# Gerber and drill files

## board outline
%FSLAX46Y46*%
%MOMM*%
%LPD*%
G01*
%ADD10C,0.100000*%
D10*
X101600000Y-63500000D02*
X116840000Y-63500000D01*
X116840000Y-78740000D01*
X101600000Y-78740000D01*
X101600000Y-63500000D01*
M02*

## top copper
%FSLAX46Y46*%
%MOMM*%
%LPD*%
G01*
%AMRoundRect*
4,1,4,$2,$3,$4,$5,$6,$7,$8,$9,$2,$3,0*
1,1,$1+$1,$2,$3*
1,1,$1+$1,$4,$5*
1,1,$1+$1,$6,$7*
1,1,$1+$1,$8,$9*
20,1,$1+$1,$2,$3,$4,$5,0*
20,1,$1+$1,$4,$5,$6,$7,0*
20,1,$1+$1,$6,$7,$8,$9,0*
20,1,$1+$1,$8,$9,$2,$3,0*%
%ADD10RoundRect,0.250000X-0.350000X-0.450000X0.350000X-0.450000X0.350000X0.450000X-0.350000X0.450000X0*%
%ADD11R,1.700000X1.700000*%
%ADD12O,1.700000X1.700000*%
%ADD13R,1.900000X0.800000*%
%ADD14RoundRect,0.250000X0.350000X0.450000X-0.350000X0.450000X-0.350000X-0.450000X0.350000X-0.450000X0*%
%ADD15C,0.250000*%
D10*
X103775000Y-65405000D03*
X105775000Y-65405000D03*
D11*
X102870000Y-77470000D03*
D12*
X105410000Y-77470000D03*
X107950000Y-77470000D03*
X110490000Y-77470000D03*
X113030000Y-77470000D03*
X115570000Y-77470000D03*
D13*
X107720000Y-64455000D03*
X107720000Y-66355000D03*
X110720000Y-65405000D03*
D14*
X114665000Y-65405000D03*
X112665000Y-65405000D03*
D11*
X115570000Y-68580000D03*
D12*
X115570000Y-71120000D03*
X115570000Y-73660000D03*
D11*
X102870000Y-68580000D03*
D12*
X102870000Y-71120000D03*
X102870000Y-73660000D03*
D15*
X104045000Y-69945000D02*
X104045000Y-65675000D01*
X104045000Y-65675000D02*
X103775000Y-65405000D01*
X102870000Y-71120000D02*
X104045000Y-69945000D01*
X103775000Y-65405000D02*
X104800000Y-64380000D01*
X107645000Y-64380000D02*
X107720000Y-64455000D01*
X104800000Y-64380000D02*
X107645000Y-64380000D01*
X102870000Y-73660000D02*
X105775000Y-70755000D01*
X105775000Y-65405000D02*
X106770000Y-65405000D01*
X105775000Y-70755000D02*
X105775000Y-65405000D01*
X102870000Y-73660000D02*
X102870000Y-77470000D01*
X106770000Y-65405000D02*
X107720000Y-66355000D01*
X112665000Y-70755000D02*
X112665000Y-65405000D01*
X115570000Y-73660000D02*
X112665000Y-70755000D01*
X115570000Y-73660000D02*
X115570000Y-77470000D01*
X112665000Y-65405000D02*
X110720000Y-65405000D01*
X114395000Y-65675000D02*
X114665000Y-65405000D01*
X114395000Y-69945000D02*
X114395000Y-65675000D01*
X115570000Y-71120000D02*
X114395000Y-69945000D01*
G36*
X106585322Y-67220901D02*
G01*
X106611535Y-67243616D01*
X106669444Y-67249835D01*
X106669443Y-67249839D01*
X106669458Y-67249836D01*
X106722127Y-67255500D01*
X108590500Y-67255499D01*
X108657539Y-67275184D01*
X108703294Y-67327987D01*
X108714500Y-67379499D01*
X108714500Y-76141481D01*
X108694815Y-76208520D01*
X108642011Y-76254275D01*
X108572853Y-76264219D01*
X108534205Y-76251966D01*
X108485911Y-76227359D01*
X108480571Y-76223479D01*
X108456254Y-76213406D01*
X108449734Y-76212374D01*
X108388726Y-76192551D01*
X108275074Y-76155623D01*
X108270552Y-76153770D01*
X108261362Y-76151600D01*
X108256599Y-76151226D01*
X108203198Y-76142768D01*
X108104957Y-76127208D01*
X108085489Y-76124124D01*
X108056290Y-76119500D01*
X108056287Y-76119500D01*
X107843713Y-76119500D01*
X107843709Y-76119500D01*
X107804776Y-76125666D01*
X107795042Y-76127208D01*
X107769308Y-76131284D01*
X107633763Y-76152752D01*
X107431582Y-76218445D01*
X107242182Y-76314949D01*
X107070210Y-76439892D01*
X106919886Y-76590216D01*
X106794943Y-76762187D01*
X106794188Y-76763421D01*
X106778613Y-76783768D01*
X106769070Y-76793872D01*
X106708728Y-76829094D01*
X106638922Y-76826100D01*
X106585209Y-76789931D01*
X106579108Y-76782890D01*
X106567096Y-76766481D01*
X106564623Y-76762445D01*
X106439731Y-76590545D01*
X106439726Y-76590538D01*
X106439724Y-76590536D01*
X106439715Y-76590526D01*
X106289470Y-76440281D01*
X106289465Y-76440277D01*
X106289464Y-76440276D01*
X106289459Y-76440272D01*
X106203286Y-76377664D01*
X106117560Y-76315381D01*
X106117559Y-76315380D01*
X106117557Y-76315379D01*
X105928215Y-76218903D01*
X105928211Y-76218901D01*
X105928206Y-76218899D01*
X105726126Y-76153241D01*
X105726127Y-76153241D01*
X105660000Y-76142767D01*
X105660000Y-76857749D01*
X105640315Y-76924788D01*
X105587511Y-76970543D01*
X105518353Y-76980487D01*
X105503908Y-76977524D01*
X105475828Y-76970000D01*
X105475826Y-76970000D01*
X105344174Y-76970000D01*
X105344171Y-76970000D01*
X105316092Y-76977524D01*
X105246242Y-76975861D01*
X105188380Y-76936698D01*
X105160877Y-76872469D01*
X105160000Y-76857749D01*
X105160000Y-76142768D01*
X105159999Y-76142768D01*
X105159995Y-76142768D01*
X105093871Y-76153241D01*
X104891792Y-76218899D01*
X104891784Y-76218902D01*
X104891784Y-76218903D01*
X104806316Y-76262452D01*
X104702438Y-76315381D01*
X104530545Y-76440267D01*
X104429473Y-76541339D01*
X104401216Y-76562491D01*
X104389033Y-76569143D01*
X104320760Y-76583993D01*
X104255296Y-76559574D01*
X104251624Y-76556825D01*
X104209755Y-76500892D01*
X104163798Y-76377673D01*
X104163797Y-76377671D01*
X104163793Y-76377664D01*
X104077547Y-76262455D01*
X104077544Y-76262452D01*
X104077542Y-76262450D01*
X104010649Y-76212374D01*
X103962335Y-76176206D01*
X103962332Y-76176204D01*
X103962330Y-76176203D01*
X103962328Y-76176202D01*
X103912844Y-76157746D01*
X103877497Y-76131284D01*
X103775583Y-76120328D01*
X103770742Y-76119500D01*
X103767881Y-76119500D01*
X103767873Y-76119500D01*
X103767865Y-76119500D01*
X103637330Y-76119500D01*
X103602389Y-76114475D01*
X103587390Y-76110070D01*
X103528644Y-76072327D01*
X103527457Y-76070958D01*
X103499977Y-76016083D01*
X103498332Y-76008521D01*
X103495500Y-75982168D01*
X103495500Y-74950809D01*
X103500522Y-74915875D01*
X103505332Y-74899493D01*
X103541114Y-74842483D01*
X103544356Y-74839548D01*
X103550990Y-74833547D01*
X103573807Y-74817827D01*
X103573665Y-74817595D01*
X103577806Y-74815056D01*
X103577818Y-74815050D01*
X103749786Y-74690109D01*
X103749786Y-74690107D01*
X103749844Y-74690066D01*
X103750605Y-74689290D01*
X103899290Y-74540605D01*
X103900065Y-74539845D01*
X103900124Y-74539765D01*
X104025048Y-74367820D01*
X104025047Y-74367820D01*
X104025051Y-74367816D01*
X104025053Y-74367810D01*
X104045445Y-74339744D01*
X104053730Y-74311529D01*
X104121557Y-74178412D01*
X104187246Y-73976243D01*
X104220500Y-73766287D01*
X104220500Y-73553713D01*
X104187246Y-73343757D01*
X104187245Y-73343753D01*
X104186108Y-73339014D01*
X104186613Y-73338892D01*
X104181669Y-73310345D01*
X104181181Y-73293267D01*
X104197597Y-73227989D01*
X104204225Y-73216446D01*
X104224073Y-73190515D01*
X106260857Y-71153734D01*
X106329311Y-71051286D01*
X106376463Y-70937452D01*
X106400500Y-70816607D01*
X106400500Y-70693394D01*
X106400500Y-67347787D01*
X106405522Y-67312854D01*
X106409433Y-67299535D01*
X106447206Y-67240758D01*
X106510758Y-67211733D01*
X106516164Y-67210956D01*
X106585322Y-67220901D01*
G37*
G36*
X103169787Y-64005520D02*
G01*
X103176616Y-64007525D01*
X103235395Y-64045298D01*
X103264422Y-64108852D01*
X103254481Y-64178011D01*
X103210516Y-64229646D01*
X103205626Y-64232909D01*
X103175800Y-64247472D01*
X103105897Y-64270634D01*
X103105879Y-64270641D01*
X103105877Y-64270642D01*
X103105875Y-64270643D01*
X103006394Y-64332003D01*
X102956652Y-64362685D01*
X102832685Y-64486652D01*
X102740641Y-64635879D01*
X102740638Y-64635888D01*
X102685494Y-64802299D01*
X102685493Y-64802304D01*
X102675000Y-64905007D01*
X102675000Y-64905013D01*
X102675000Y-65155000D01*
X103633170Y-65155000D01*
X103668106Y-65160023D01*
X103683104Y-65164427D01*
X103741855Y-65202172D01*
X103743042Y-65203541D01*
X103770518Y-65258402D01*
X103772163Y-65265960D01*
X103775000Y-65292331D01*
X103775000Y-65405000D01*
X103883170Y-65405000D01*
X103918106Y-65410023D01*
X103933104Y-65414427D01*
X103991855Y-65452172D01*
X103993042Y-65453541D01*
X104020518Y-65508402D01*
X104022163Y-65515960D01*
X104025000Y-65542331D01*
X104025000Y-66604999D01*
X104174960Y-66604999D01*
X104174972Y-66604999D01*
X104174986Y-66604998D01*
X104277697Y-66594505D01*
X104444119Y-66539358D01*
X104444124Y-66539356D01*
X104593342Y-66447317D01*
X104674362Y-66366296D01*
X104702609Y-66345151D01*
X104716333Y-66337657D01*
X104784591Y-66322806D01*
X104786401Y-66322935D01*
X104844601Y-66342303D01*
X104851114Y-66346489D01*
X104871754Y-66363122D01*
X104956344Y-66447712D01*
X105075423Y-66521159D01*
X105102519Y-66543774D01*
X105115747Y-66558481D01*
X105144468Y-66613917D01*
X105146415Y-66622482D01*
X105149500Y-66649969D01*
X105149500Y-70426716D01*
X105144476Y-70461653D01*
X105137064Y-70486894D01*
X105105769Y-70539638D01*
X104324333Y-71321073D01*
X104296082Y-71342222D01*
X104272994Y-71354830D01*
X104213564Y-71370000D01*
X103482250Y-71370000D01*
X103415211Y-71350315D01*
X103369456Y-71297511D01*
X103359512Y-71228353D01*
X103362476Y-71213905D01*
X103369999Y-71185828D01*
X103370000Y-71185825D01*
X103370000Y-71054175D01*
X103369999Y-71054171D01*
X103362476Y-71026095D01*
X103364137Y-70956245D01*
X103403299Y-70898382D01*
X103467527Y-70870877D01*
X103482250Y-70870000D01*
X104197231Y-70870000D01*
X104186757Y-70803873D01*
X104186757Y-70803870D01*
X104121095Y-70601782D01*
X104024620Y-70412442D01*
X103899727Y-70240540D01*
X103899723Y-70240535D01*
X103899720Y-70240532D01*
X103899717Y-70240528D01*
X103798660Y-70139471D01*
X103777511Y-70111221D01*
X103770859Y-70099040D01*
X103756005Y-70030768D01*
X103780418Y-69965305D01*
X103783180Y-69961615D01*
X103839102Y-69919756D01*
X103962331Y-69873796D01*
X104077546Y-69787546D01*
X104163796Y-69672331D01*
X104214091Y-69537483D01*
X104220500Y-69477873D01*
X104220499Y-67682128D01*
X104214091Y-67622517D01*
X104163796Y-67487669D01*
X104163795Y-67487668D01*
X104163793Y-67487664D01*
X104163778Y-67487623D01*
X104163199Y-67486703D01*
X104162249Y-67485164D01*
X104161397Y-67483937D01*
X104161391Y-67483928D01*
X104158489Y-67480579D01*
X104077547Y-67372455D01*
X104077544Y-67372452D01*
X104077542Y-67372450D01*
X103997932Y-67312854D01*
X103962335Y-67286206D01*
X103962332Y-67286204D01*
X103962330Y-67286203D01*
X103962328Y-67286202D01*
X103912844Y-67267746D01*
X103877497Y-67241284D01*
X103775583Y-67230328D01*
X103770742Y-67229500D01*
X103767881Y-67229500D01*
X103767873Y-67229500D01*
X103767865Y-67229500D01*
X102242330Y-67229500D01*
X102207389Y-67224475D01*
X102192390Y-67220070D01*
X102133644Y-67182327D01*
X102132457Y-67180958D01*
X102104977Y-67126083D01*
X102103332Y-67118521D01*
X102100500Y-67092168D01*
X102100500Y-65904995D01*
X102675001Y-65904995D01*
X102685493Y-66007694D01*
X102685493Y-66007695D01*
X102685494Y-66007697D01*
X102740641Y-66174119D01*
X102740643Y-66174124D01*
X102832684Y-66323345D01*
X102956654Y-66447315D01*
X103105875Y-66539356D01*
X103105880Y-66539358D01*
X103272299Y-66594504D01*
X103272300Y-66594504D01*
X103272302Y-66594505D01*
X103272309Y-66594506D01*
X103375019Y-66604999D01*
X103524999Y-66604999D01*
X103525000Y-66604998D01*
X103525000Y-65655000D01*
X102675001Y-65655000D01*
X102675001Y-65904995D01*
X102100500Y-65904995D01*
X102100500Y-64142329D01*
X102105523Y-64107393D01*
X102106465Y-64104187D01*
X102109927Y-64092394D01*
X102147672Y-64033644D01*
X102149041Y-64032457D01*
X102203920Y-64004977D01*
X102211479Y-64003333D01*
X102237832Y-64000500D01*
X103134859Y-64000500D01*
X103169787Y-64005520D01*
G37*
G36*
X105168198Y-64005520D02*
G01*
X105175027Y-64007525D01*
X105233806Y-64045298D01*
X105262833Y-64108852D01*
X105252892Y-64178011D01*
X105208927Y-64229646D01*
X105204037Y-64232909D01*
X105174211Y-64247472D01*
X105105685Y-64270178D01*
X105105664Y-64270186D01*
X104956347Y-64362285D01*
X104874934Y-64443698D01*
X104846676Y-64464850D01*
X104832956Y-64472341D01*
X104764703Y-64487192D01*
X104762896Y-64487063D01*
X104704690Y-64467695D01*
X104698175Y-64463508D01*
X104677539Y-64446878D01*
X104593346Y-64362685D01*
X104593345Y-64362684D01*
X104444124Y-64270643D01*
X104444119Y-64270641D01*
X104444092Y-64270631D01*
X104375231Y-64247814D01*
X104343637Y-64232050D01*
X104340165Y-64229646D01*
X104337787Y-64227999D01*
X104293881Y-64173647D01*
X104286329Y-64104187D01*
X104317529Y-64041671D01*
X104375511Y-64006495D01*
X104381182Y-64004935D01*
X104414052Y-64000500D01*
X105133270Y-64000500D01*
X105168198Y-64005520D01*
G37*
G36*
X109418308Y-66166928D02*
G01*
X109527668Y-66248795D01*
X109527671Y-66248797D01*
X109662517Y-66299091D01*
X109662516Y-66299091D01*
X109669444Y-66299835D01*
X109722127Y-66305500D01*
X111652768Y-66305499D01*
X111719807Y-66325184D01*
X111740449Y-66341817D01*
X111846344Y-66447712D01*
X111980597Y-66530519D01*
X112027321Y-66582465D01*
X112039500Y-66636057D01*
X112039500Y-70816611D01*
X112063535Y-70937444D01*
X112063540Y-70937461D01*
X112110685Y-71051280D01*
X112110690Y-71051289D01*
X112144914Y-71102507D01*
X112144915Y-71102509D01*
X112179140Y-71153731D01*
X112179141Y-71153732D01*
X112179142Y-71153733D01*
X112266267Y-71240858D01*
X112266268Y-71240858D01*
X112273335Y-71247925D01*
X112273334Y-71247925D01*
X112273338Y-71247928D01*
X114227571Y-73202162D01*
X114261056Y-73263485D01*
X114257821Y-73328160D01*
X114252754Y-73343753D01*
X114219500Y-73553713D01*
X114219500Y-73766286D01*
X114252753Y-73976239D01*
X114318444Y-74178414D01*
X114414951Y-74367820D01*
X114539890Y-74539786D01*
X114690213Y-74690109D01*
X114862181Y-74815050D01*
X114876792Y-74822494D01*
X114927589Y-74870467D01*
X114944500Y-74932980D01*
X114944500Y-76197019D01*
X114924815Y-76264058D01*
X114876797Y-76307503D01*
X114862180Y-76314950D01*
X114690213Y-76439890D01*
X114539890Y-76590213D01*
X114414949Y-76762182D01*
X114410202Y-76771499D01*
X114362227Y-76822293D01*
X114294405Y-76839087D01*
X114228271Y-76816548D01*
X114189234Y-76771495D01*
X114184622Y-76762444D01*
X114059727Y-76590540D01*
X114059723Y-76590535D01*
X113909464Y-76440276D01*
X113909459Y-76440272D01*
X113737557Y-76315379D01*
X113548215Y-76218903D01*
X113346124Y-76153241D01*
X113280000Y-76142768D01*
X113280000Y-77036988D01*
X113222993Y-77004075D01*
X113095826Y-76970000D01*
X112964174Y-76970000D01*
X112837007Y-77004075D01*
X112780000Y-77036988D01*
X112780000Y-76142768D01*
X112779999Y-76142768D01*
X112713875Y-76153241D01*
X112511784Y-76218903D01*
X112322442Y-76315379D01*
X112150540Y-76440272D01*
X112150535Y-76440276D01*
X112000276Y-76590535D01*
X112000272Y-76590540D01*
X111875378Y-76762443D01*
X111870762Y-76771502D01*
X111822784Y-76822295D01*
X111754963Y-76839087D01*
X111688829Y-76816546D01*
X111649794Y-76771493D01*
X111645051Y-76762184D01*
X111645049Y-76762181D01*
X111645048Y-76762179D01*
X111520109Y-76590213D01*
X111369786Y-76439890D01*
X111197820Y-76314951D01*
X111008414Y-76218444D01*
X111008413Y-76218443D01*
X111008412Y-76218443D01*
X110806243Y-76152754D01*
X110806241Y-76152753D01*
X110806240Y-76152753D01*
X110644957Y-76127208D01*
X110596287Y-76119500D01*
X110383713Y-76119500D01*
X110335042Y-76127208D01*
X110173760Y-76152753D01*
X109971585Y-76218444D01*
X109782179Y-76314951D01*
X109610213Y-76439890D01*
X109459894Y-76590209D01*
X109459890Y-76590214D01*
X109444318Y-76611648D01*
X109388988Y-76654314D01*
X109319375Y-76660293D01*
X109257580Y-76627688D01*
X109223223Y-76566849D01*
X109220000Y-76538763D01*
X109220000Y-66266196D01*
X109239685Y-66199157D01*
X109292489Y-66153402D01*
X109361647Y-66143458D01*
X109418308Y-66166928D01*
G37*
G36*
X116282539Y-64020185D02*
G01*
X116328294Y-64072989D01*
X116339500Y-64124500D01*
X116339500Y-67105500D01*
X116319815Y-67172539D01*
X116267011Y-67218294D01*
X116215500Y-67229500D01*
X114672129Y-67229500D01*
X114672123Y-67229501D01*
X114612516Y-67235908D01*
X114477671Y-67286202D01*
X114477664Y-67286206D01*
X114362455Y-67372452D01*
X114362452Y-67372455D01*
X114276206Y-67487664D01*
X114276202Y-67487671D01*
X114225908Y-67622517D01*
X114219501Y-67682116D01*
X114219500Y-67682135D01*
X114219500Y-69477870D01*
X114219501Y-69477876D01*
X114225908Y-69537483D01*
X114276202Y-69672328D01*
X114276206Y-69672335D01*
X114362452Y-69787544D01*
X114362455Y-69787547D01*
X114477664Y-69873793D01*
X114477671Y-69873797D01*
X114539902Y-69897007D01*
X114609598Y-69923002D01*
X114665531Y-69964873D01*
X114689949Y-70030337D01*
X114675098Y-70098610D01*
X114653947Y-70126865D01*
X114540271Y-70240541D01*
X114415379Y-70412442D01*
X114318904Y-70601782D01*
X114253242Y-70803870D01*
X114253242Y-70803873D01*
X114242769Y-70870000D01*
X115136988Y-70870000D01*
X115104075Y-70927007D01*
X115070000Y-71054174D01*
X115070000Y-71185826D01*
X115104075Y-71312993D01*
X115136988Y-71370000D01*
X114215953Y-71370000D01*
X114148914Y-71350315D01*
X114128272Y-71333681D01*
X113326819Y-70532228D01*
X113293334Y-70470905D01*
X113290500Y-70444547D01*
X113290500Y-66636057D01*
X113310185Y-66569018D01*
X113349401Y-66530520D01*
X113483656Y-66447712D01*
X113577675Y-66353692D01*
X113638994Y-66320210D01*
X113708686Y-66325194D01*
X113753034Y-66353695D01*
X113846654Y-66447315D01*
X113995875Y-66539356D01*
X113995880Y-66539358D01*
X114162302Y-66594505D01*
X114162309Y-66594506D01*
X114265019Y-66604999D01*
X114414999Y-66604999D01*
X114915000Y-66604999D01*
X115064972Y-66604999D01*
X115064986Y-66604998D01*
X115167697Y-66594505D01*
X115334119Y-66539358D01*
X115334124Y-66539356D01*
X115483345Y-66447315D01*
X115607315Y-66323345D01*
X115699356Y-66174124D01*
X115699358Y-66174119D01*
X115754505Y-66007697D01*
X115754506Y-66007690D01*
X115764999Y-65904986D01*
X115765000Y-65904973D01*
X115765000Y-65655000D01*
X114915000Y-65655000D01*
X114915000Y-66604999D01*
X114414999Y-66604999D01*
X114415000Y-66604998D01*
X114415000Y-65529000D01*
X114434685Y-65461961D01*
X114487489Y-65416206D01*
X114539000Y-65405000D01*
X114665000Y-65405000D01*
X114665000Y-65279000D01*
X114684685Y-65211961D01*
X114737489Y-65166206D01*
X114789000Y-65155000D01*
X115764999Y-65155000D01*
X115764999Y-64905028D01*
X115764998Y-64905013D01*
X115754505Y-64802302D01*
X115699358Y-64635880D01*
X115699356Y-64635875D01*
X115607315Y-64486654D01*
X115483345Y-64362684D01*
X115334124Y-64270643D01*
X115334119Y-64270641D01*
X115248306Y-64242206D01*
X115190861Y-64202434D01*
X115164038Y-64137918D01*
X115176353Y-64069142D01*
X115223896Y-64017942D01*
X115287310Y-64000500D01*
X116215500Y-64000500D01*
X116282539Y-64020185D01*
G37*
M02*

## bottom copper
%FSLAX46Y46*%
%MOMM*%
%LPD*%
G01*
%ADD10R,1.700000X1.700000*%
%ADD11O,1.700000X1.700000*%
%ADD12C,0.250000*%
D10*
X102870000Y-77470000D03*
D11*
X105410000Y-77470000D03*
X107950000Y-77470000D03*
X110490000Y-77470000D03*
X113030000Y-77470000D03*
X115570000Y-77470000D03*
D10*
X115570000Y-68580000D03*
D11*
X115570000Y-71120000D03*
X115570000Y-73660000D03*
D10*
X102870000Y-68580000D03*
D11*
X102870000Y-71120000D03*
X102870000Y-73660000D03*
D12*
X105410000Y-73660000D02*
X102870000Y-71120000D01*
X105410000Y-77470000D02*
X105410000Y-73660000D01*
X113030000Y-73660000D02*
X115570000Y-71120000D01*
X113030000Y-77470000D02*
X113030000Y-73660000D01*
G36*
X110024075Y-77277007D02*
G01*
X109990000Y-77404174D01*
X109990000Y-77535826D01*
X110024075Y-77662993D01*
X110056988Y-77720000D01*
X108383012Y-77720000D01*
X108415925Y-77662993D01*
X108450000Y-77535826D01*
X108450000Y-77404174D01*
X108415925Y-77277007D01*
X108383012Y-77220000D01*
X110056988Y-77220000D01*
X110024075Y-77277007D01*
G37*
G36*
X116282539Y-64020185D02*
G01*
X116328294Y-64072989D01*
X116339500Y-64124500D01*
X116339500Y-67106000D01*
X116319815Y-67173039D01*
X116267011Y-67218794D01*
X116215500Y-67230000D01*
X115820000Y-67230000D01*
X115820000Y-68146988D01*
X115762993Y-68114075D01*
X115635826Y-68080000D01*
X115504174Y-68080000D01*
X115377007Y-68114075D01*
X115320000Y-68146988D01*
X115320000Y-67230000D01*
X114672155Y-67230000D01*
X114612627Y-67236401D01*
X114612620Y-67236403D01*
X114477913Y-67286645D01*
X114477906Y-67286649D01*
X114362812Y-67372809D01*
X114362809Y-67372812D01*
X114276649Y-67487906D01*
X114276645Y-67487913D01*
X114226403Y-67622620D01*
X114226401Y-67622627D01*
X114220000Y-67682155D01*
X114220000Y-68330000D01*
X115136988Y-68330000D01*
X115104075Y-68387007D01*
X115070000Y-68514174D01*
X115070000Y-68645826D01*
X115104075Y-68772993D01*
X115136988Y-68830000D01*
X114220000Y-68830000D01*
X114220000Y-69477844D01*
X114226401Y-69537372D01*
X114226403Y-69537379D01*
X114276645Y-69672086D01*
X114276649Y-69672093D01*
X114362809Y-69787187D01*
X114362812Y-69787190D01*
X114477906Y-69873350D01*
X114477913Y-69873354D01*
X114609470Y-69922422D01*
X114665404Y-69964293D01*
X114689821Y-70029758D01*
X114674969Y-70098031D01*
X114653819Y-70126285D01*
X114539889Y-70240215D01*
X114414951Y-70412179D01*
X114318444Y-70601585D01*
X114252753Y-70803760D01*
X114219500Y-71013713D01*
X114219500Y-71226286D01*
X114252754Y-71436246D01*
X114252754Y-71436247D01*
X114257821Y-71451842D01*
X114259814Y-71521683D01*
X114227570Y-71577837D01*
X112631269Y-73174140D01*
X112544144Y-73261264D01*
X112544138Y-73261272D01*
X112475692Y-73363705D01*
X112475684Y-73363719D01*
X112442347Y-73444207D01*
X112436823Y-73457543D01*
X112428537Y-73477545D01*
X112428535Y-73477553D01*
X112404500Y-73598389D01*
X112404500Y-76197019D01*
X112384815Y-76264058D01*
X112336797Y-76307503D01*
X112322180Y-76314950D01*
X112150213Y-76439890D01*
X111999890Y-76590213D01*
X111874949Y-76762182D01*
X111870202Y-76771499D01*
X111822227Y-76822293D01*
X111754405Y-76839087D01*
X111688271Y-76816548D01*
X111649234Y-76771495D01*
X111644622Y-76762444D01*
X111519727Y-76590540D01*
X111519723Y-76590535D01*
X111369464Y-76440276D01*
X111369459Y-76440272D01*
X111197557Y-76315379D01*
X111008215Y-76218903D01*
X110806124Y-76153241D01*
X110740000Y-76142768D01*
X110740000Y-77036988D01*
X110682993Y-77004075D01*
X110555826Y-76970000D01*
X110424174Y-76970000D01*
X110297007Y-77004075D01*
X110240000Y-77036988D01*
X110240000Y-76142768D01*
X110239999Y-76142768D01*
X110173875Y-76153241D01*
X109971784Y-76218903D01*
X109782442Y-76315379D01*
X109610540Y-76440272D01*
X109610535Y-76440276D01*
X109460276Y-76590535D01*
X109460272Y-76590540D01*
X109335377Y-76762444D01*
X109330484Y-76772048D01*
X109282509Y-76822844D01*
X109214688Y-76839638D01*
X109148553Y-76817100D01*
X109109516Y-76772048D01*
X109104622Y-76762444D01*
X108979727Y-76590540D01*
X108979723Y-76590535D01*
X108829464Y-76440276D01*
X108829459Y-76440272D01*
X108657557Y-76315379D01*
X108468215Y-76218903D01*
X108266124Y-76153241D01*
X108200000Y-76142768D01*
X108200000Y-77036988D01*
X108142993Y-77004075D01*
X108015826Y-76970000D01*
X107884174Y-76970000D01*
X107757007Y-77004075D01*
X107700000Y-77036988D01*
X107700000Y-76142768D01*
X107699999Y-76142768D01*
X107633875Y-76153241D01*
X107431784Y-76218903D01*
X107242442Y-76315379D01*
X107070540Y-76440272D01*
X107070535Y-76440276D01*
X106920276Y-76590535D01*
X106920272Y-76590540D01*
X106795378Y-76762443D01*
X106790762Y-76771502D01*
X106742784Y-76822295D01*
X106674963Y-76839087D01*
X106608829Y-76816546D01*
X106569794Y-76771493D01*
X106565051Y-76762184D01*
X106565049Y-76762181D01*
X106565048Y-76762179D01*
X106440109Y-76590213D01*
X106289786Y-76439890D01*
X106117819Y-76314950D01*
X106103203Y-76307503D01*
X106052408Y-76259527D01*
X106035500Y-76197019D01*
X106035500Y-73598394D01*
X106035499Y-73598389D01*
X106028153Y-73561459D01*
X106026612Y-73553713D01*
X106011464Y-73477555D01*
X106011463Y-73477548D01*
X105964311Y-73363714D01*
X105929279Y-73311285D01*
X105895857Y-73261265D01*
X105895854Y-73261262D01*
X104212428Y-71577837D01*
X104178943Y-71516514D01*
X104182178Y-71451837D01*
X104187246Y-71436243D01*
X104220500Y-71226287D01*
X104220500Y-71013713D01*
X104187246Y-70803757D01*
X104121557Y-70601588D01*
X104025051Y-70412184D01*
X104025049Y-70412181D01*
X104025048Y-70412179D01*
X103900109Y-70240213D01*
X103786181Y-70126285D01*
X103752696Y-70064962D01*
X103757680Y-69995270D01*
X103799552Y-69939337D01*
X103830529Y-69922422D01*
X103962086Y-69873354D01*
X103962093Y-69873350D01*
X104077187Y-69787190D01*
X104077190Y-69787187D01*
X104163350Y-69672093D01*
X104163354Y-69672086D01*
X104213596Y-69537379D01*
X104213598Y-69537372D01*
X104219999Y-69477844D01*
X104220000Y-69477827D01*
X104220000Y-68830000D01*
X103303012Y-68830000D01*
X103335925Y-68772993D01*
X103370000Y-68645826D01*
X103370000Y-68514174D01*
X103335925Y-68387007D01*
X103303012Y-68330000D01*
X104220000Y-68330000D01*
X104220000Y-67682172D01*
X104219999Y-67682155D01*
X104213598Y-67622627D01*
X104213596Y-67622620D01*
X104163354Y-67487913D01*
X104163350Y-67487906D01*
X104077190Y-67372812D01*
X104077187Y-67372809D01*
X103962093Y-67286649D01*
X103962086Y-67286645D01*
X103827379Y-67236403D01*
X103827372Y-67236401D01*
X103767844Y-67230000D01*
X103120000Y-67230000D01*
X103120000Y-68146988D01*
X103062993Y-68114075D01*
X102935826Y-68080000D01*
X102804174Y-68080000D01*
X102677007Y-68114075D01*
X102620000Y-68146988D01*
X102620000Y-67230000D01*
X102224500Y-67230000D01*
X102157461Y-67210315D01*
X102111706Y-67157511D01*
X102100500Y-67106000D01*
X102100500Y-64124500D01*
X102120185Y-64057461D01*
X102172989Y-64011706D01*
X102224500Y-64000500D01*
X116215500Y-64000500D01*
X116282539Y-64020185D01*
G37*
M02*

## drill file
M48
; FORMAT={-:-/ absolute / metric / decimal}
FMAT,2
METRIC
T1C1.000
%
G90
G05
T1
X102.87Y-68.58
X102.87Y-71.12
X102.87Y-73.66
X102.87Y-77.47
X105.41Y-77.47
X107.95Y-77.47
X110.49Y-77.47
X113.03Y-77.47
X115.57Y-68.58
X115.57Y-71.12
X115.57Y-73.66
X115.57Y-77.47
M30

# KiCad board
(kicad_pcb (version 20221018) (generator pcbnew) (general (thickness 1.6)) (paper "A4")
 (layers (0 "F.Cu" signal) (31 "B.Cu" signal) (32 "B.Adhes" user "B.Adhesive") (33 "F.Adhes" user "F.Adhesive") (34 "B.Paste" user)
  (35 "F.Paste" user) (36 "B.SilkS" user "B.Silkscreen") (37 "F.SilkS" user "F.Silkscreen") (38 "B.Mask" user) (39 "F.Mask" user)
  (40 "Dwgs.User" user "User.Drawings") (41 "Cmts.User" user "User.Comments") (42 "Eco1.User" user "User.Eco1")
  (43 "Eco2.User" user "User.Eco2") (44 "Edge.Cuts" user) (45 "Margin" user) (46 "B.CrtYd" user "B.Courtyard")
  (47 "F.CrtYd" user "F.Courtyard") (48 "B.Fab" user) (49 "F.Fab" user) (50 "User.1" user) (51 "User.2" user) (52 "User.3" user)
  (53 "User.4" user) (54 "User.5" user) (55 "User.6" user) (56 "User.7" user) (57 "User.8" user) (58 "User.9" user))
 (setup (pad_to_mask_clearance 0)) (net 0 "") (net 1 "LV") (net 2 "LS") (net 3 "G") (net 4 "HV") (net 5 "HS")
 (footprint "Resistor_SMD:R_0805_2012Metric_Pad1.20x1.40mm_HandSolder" (layer "F.Cu") (at 104.775 65.405)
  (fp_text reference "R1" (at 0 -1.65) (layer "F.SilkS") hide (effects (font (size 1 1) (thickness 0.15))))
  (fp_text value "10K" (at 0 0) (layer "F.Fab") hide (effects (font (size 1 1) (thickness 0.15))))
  (pad "1" smd roundrect (at -1 0) (size 1.2 1.4) (layers "F.Cu" "F.Paste" "F.Mask") (roundrect_rratio 0.208333) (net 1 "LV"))
  (pad "2" smd roundrect (at 1 0) (size 1.2 1.4) (layers "F.Cu" "F.Paste" "F.Mask") (roundrect_rratio 0.208333) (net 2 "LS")))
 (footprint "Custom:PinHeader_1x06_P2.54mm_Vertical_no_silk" (layer "F.Cu") (at 102.87 77.47 90)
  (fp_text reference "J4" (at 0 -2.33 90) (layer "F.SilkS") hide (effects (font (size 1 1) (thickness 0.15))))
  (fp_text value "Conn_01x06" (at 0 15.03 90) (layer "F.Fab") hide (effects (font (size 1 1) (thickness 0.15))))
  (pad "1" thru_hole rect (at 0 0 90) (size 1.7 1.7) (drill 1) (layers "*.Cu" "*.Mask") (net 2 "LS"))
  (pad "2" thru_hole oval (at 0 2.54 90) (size 1.7 1.7) (drill 1) (layers "*.Cu" "*.Mask") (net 1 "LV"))
  (pad "3" thru_hole oval (at 0 5.08 90) (size 1.7 1.7) (drill 1) (layers "*.Cu" "*.Mask") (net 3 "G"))
  (pad "4" thru_hole oval (at 0 7.62 90) (size 1.7 1.7) (drill 1) (layers "*.Cu" "*.Mask") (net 3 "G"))
  (pad "5" thru_hole oval (at 0 10.16 90) (size 1.7 1.7) (drill 1) (layers "*.Cu" "*.Mask") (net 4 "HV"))
  (pad "6" thru_hole oval (at 0 12.7 90) (size 1.7 1.7) (drill 1) (layers "*.Cu" "*.Mask") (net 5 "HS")))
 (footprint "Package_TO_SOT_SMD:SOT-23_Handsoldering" (layer "F.Cu") (at 109.22 65.405)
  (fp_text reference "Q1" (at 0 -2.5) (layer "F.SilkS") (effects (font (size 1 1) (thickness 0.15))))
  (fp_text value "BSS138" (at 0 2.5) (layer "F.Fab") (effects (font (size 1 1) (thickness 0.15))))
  (pad "1" smd rect (at -1.5 -0.95) (size 1.9 0.8) (layers "F.Cu" "F.Paste" "F.Mask") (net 1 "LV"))
  (pad "2" smd rect (at -1.5 0.95) (size 1.9 0.8) (layers "F.Cu" "F.Paste" "F.Mask") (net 2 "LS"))
  (pad "3" smd rect (at 1.5 0) (size 1.9 0.8) (layers "F.Cu" "F.Paste" "F.Mask") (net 5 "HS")))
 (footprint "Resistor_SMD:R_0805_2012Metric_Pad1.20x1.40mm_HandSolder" (layer "F.Cu") (at 113.665 65.405 180)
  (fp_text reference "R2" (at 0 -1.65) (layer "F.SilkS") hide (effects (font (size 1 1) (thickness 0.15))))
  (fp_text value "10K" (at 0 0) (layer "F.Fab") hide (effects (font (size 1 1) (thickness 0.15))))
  (pad "1" smd roundrect (at -1 0 180) (size 1.2 1.4) (layers "F.Cu" "F.Paste" "F.Mask") (roundrect_rratio 0.208333) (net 4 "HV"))
  (pad "2" smd roundrect (at 1 0 180) (size 1.2 1.4) (layers "F.Cu" "F.Paste" "F.Mask") (roundrect_rratio 0.208333) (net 5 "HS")))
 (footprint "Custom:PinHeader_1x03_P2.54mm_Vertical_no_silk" (layer "F.Cu") (at 115.57 68.58)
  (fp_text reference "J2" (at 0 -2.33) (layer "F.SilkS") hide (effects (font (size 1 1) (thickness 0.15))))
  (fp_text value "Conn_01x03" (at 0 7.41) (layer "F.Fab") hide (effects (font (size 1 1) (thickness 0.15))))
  (pad "1" thru_hole rect (at 0 0) (size 1.7 1.7) (drill 1) (layers "*.Cu" "*.Mask") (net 3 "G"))
  (pad "2" thru_hole oval (at 0 2.54) (size 1.7 1.7) (drill 1) (layers "*.Cu" "*.Mask") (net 4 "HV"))
  (pad "3" thru_hole oval (at 0 5.08) (size 1.7 1.7) (drill 1) (layers "*.Cu" "*.Mask") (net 5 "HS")))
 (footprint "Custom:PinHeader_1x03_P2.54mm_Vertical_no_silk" (layer "F.Cu") (at 102.87 68.58)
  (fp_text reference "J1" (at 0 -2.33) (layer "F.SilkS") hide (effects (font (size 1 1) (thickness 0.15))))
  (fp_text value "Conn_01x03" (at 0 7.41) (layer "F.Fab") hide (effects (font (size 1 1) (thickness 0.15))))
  (pad "1" thru_hole rect (at 0 0) (size 1.7 1.7) (drill 1) (layers "*.Cu" "*.Mask") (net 3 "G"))
  (pad "2" thru_hole oval (at 0 2.54) (size 1.7 1.7) (drill 1) (layers "*.Cu" "*.Mask") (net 1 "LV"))
  (pad "3" thru_hole oval (at 0 5.08) (size 1.7 1.7) (drill 1) (layers "*.Cu" "*.Mask") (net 2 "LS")))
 (gr_rect (start 101.6 63.5) (end 116.84 78.74) (stroke (width 0.1) (type default)) (fill none) (layer "Edge.Cuts"))
 (segment (start 104.045 69.945) (end 104.045 65.675) (width 0.25) (layer "F.Cu") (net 1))
 (segment (start 104.045 65.675) (end 103.775 65.405) (width 0.25) (layer "F.Cu") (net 1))
 (segment (start 102.87 71.12) (end 104.045 69.945) (width 0.25) (layer "F.Cu") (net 1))
 (segment (start 103.775 65.405) (end 104.8 64.38) (width 0.25) (layer "F.Cu") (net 1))
 (segment (start 107.645 64.38) (end 107.72 64.455) (width 0.25) (layer "F.Cu") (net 1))
 (segment (start 104.8 64.38) (end 107.645 64.38) (width 0.25) (layer "F.Cu") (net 1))
 (segment (start 105.41 73.66) (end 102.87 71.12) (width 0.25) (layer "B.Cu") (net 1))
 (segment (start 105.41 77.47) (end 105.41 73.66) (width 0.25) (layer "B.Cu") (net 1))
 (segment (start 102.87 73.66) (end 105.775 70.755) (width 0.25) (layer "F.Cu") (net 2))
 (segment (start 105.775 65.405) (end 106.77 65.405) (width 0.25) (layer "F.Cu") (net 2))
 (segment (start 105.775 70.755) (end 105.775 65.405) (width 0.25) (layer "F.Cu") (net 2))
 (segment (start 102.87 73.66) (end 102.87 77.47) (width 0.25) (layer "F.Cu") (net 2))
 (segment (start 106.77 65.405) (end 107.72 66.355) (width 0.25) (layer "F.Cu") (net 2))
 (segment (start 112.665 70.755) (end 112.665 65.405) (width 0.25) (layer "F.Cu") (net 5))
 (segment (start 115.57 73.66) (end 112.665 70.755) (width 0.25) (layer "F.Cu") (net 5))
 (segment (start 115.57 73.66) (end 115.57 77.47) (width 0.25) (layer "F.Cu") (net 5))
 (segment (start 112.665 65.405) (end 110.72 65.405) (width 0.25) (layer "F.Cu") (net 5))
 (segment (start 114.395 65.675) (end 114.665 65.405) (width 0.25) (layer "F.Cu") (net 4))
 (segment (start 114.395 69.945) (end 114.395 65.675) (width 0.25) (layer "F.Cu") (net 4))
 (segment (start 115.57 71.12) (end 114.395 69.945) (width 0.25) (layer "F.Cu") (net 4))
 (segment (start 113.03 73.66) (end 115.57 71.12) (width 0.25) (layer "B.Cu") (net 4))
 (segment (start 113.03 77.47) (end 113.03 73.66) (width 0.25) (layer "B.Cu") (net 4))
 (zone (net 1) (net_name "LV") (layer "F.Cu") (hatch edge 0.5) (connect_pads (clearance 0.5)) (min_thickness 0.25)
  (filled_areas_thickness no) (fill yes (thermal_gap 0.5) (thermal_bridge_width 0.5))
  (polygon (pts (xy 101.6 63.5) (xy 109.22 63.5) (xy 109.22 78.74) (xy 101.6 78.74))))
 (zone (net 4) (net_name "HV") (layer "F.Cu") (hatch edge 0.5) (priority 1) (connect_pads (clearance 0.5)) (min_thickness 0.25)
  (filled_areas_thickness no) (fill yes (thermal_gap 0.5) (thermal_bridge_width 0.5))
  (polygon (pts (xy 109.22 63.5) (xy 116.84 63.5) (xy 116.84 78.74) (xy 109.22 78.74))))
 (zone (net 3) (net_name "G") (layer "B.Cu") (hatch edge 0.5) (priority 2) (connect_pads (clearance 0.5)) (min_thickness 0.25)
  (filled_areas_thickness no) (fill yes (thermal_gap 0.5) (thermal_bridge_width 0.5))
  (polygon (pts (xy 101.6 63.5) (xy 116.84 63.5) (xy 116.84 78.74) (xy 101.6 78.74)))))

